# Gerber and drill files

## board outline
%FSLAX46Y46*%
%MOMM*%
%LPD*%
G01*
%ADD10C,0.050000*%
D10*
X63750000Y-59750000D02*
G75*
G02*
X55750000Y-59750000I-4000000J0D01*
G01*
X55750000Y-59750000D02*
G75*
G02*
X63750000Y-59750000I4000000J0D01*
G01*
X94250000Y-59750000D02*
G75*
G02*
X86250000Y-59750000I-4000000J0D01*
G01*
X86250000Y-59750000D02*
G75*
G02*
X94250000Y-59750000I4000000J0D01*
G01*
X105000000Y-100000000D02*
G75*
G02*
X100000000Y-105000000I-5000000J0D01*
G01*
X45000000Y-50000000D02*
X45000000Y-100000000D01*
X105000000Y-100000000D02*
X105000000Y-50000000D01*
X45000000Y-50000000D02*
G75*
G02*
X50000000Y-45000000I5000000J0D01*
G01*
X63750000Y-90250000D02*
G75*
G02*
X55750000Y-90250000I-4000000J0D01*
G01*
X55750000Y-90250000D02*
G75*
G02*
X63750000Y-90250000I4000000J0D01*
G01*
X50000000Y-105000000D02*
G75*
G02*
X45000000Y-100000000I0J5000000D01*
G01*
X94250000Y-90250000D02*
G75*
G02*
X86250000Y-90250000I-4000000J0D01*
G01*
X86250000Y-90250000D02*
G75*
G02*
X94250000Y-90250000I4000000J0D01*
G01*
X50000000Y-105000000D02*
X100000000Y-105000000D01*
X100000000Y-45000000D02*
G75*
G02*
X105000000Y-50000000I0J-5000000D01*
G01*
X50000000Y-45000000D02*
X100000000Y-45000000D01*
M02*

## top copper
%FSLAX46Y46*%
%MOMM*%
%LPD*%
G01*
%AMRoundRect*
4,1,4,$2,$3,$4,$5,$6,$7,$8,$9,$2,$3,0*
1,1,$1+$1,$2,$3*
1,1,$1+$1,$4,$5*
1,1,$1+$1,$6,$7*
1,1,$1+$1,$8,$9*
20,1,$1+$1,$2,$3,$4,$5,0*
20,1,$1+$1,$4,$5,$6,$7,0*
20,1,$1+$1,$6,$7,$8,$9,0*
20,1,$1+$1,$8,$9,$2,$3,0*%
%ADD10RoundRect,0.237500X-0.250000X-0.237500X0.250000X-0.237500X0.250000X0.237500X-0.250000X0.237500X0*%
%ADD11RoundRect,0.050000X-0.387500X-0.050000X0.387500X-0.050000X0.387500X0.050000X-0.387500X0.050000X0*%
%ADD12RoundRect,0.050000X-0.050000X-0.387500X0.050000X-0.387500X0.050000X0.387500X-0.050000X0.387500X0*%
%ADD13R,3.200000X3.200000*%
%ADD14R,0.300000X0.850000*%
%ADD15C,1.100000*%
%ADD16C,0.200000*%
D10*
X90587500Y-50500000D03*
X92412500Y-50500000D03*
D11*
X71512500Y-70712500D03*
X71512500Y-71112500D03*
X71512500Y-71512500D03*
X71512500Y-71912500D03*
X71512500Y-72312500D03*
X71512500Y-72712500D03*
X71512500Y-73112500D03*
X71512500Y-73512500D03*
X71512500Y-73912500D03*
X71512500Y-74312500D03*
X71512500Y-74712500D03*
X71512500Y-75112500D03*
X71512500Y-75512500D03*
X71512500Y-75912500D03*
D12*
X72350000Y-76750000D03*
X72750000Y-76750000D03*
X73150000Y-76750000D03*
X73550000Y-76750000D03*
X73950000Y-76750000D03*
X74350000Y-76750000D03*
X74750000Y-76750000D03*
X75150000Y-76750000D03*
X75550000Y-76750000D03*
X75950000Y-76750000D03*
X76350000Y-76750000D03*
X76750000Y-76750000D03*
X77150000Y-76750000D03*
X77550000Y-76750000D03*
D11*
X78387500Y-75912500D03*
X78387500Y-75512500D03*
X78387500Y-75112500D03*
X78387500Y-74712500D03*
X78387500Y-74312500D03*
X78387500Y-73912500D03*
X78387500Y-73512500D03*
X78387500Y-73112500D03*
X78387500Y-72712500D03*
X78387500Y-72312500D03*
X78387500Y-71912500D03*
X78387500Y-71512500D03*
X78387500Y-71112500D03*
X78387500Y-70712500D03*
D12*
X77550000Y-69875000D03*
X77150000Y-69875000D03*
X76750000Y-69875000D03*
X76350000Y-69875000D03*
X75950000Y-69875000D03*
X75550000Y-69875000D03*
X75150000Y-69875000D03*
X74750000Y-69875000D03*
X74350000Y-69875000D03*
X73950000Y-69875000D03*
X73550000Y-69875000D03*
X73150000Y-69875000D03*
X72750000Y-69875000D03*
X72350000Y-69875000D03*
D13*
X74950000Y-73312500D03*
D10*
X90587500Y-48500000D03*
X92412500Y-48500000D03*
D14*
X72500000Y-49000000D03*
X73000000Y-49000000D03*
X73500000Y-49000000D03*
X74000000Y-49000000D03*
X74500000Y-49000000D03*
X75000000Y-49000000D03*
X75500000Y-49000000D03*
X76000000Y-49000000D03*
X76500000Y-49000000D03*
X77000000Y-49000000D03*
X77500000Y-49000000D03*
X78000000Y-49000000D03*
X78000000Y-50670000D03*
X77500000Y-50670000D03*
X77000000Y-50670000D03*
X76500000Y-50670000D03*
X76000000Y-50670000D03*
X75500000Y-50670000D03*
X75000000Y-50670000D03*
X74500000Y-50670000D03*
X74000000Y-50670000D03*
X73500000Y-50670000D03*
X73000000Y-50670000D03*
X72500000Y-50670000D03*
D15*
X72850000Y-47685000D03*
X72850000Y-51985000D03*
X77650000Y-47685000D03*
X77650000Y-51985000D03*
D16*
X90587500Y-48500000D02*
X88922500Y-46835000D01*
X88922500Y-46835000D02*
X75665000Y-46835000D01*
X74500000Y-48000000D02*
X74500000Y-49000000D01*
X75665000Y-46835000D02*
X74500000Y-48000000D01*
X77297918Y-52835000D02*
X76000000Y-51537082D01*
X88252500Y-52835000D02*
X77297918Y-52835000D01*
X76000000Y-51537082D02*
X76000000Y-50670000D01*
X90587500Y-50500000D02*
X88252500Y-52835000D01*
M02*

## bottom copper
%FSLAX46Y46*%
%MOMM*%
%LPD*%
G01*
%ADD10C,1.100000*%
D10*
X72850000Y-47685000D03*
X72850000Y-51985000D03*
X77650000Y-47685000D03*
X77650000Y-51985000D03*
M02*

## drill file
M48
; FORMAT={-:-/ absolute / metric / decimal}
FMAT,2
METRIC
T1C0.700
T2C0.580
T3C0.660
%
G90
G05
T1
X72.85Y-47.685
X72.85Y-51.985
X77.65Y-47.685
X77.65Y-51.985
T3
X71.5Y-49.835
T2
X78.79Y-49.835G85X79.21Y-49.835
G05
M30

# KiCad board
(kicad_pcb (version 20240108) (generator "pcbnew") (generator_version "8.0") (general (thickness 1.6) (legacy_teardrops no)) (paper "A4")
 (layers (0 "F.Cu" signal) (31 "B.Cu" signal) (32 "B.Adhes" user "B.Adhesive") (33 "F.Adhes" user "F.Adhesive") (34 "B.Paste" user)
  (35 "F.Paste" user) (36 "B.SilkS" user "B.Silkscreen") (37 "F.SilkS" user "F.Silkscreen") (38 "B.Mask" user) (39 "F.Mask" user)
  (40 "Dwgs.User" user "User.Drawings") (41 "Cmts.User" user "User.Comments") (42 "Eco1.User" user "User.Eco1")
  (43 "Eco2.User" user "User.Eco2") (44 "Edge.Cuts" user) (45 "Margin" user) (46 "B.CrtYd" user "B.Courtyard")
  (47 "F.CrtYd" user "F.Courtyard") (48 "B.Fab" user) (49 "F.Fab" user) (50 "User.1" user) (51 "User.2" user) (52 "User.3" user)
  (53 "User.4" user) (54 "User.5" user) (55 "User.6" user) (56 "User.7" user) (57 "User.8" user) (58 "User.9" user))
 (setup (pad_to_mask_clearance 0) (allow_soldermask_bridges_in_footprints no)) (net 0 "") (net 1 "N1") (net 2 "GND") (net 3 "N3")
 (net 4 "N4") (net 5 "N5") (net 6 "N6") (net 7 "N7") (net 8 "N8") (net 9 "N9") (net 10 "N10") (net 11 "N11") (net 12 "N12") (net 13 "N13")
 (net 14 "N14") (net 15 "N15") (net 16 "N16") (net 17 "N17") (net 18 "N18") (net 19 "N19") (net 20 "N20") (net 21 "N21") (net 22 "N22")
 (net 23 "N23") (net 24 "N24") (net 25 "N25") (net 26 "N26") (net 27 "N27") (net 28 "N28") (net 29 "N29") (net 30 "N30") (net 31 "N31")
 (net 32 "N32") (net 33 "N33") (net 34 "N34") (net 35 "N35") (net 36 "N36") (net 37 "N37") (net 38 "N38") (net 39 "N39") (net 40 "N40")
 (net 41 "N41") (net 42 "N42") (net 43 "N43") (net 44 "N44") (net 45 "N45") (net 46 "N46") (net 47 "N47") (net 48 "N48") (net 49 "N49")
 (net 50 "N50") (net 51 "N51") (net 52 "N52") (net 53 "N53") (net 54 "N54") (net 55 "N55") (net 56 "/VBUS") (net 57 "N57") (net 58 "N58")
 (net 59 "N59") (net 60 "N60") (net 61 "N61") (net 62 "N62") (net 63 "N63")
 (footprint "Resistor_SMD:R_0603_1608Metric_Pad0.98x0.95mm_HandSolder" (layer "F.Cu") (at 91.5 50.5)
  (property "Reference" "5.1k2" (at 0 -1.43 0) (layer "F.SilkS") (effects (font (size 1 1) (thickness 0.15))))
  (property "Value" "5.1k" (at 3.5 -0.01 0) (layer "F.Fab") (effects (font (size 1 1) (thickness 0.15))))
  (pad "1" smd roundrect (at -0.9125 0) (size 0.975 0.95) (layers "F.Cu" "F.Paste" "F.Mask") (roundrect_rratio 0.25) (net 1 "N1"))
  (pad "2" smd roundrect (at 0.9125 0) (size 0.975 0.95) (layers "F.Cu" "F.Paste" "F.Mask") (roundrect_rratio 0.25) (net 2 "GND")))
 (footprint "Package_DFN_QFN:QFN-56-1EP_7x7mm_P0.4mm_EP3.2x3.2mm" (layer "F.Cu") (at 74.95 73.3125)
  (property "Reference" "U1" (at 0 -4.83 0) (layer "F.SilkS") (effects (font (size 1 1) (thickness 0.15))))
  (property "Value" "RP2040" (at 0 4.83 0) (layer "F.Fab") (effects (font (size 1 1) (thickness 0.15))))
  (pad "" smd roundrect (at -0.8 -0.8) (size 1.29 1.29) (layers "F.Paste") (roundrect_rratio 0.193798))
  (pad "" smd roundrect (at -0.8 0.8) (size 1.29 1.29) (layers "F.Paste") (roundrect_rratio 0.193798))
  (pad "" smd roundrect (at 0.8 -0.8) (size 1.29 1.29) (layers "F.Paste") (roundrect_rratio 0.193798))
  (pad "" smd roundrect (at 0.8 0.8) (size 1.29 1.29) (layers "F.Paste") (roundrect_rratio 0.193798))
  (pad "1" smd roundrect (at -3.4375 -2.6) (size 0.875 0.2) (layers "F.Cu" "F.Paste" "F.Mask") (roundrect_rratio 0.25) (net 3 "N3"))
  (pad "2" smd roundrect (at -3.4375 -2.2) (size 0.875 0.2) (layers "F.Cu" "F.Paste" "F.Mask") (roundrect_rratio 0.25) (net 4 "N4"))
  (pad "3" smd roundrect (at -3.4375 -1.8) (size 0.875 0.2) (layers "F.Cu" "F.Paste" "F.Mask") (roundrect_rratio 0.25) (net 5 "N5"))
  (pad "4" smd roundrect (at -3.4375 -1.4) (size 0.875 0.2) (layers "F.Cu" "F.Paste" "F.Mask") (roundrect_rratio 0.25) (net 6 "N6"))
  (pad "5" smd roundrect (at -3.4375 -1) (size 0.875 0.2) (layers "F.Cu" "F.Paste" "F.Mask") (roundrect_rratio 0.25) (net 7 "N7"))
  (pad "6" smd roundrect (at -3.4375 -0.6) (size 0.875 0.2) (layers "F.Cu" "F.Paste" "F.Mask") (roundrect_rratio 0.25) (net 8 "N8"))
  (pad "7" smd roundrect (at -3.4375 -0.2) (size 0.875 0.2) (layers "F.Cu" "F.Paste" "F.Mask") (roundrect_rratio 0.25) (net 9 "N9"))
  (pad "8" smd roundrect (at -3.4375 0.2) (size 0.875 0.2) (layers "F.Cu" "F.Paste" "F.Mask") (roundrect_rratio 0.25) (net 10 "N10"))
  (pad "9" smd roundrect (at -3.4375 0.6) (size 0.875 0.2) (layers "F.Cu" "F.Paste" "F.Mask") (roundrect_rratio 0.25) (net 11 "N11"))
  (pad "10" smd roundrect (at -3.4375 1) (size 0.875 0.2) (layers "F.Cu" "F.Paste" "F.Mask") (roundrect_rratio 0.25) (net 3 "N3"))
  (pad "11" smd roundrect (at -3.4375 1.4) (size 0.875 0.2) (layers "F.Cu" "F.Paste" "F.Mask") (roundrect_rratio 0.25) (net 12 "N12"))
  (pad "12" smd roundrect (at -3.4375 1.8) (size 0.875 0.2) (layers "F.Cu" "F.Paste" "F.Mask") (roundrect_rratio 0.25) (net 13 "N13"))
  (pad "13" smd roundrect (at -3.4375 2.2) (size 0.875 0.2) (layers "F.Cu" "F.Paste" "F.Mask") (roundrect_rratio 0.25) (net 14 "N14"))
  (pad "14" smd roundrect (at -3.4375 2.6) (size 0.875 0.2) (layers "F.Cu" "F.Paste" "F.Mask") (roundrect_rratio 0.25) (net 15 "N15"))
  (pad "15" smd roundrect (at -2.6 3.4375) (size 0.2 0.875) (layers "F.Cu" "F.Paste" "F.Mask") (roundrect_rratio 0.25) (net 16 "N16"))
  (pad "16" smd roundrect (at -2.2 3.4375) (size 0.2 0.875) (layers "F.Cu" "F.Paste" "F.Mask") (roundrect_rratio 0.25) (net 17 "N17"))
  (pad "17" smd roundrect (at -1.8 3.4375) (size 0.2 0.875) (layers "F.Cu" "F.Paste" "F.Mask") (roundrect_rratio 0.25) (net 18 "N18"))
  (pad "18" smd roundrect (at -1.4 3.4375) (size 0.2 0.875) (layers "F.Cu" "F.Paste" "F.Mask") (roundrect_rratio 0.25) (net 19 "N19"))
  (pad "19" smd roundrect (at -1 3.4375) (size 0.2 0.875) (layers "F.Cu" "F.Paste" "F.Mask") (roundrect_rratio 0.25) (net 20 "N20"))
  (pad "20" smd roundrect (at -0.6 3.4375) (size 0.2 0.875) (layers "F.Cu" "F.Paste" "F.Mask") (roundrect_rratio 0.25) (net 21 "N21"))
  (pad "21" smd roundrect (at -0.2 3.4375) (size 0.2 0.875) (layers "F.Cu" "F.Paste" "F.Mask") (roundrect_rratio 0.25) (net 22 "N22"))
  (pad "22" smd roundrect (at 0.2 3.4375) (size 0.2 0.875) (layers "F.Cu" "F.Paste" "F.Mask") (roundrect_rratio 0.25) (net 3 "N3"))
  (pad "23" smd roundrect (at 0.6 3.4375) (size 0.2 0.875) (layers "F.Cu" "F.Paste" "F.Mask") (roundrect_rratio 0.25) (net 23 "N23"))
  (pad "24" smd roundrect (at 1 3.4375) (size 0.2 0.875) (layers "F.Cu" "F.Paste" "F.Mask") (roundrect_rratio 0.25) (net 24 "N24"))
  (pad "25" smd roundrect (at 1.4 3.4375) (size 0.2 0.875) (layers "F.Cu" "F.Paste" "F.Mask") (roundrect_rratio 0.25) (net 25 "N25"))
  (pad "26" smd roundrect (at 1.8 3.4375) (size 0.2 0.875) (layers "F.Cu" "F.Paste" "F.Mask") (roundrect_rratio 0.25) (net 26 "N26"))
  (pad "27" smd roundrect (at 2.2 3.4375) (size 0.2 0.875) (layers "F.Cu" "F.Paste" "F.Mask") (roundrect_rratio 0.25) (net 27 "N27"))
  (pad "28" smd roundrect (at 2.6 3.4375) (size 0.2 0.875) (layers "F.Cu" "F.Paste" "F.Mask") (roundrect_rratio 0.25) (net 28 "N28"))
  (pad "29" smd roundrect (at 3.4375 2.6) (size 0.875 0.2) (layers "F.Cu" "F.Paste" "F.Mask") (roundrect_rratio 0.25) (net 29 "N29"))
  (pad "30" smd roundrect (at 3.4375 2.2) (size 0.875 0.2) (layers "F.Cu" "F.Paste" "F.Mask") (roundrect_rratio 0.25) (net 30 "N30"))
  (pad "31" smd roundrect (at 3.4375 1.8) (size 0.875 0.2) (layers "F.Cu" "F.Paste" "F.Mask") (roundrect_rratio 0.25) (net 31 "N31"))
  (pad "32" smd roundrect (at 3.4375 1.4) (size 0.875 0.2) (layers "F.Cu" "F.Paste" "F.Mask") (roundrect_rratio 0.25) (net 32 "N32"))
  (pad "33" smd roundrect (at 3.4375 1) (size 0.875 0.2) (layers "F.Cu" "F.Paste" "F.Mask") (roundrect_rratio 0.25) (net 3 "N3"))
  (pad "34" smd roundrect (at 3.4375 0.6) (size 0.875 0.2) (layers "F.Cu" "F.Paste" "F.Mask") (roundrect_rratio 0.25) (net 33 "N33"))
  (pad "35" smd roundrect (at 3.4375 0.2) (size 0.875 0.2) (layers "F.Cu" "F.Paste" "F.Mask") (roundrect_rratio 0.25) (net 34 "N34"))
  (pad "36" smd roundrect (at 3.4375 -0.2) (size 0.875 0.2) (layers "F.Cu" "F.Paste" "F.Mask") (roundrect_rratio 0.25) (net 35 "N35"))
  (pad "37" smd roundrect (at 3.4375 -0.6) (size 0.875 0.2) (layers "F.Cu" "F.Paste" "F.Mask") (roundrect_rratio 0.25) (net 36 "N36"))
  (pad "38" smd roundrect (at 3.4375 -1) (size 0.875 0.2) (layers "F.Cu" "F.Paste" "F.Mask") (roundrect_rratio 0.25) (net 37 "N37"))
  (pad "39" smd roundrect (at 3.4375 -1.4) (size 0.875 0.2) (layers "F.Cu" "F.Paste" "F.Mask") (roundrect_rratio 0.25) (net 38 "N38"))
  (pad "40" smd roundrect (at 3.4375 -1.8) (size 0.875 0.2) (layers "F.Cu" "F.Paste" "F.Mask") (roundrect_rratio 0.25) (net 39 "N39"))
  (pad "41" smd roundrect (at 3.4375 -2.2) (size 0.875 0.2) (layers "F.Cu" "F.Paste" "F.Mask") (roundrect_rratio 0.25) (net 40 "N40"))
  (pad "42" smd roundrect (at 3.4375 -2.6) (size 0.875 0.2) (layers "F.Cu" "F.Paste" "F.Mask") (roundrect_rratio 0.25) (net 3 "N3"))
  (pad "43" smd roundrect (at 2.6 -3.4375) (size 0.2 0.875) (layers "F.Cu" "F.Paste" "F.Mask") (roundrect_rratio 0.25) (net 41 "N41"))
  (pad "44" smd roundrect (at 2.2 -3.4375) (size 0.2 0.875) (layers "F.Cu" "F.Paste" "F.Mask") (roundrect_rratio 0.25) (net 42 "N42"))
  (pad "45" smd roundrect (at 1.8 -3.4375) (size 0.2 0.875) (layers "F.Cu" "F.Paste" "F.Mask") (roundrect_rratio 0.25) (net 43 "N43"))
  (pad "46" smd roundrect (at 1.4 -3.4375) (size 0.2 0.875) (layers "F.Cu" "F.Paste" "F.Mask") (roundrect_rratio 0.25) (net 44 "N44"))
  (pad "47" smd roundrect (at 1 -3.4375) (size 0.2 0.875) (layers "F.Cu" "F.Paste" "F.Mask") (roundrect_rratio 0.25) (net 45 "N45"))
  (pad "48" smd roundrect (at 0.6 -3.4375) (size 0.2 0.875) (layers "F.Cu" "F.Paste" "F.Mask") (roundrect_rratio 0.25) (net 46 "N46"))
  (pad "49" smd roundrect (at 0.2 -3.4375) (size 0.2 0.875) (layers "F.Cu" "F.Paste" "F.Mask") (roundrect_rratio 0.25) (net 3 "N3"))
  (pad "50" smd roundrect (at -0.2 -3.4375) (size 0.2 0.875) (layers "F.Cu" "F.Paste" "F.Mask") (roundrect_rratio 0.25) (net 23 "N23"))
  (pad "51" smd roundrect (at -0.6 -3.4375) (size 0.2 0.875) (layers "F.Cu" "F.Paste" "F.Mask") (roundrect_rratio 0.25) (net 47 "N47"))
  (pad "52" smd roundrect (at -1 -3.4375) (size 0.2 0.875) (layers "F.Cu" "F.Paste" "F.Mask") (roundrect_rratio 0.25) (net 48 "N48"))
  (pad "53" smd roundrect (at -1.4 -3.4375) (size 0.2 0.875) (layers "F.Cu" "F.Paste" "F.Mask") (roundrect_rratio 0.25) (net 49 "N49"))
  (pad "54" smd roundrect (at -1.8 -3.4375) (size 0.2 0.875) (layers "F.Cu" "F.Paste" "F.Mask") (roundrect_rratio 0.25) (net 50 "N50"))
  (pad "55" smd roundrect (at -2.2 -3.4375) (size 0.2 0.875) (layers "F.Cu" "F.Paste" "F.Mask") (roundrect_rratio 0.25) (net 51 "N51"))
  (pad "56" smd roundrect (at -2.6 -3.4375) (size 0.2 0.875) (layers "F.Cu" "F.Paste" "F.Mask") (roundrect_rratio 0.25) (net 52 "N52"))
  (pad "57" smd rect (at 0 0) (size 3.2 3.2) (layers "F.Cu" "F.Mask") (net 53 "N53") (zone_connect 2)))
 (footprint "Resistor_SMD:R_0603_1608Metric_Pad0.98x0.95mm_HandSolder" (layer "F.Cu") (at 91.5 48.5)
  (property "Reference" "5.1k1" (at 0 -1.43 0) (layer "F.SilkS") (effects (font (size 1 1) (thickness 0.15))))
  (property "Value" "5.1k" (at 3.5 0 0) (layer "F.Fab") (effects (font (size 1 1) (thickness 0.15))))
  (pad "1" smd roundrect (at -0.9125 0) (size 0.975 0.95) (layers "F.Cu" "F.Paste" "F.Mask") (roundrect_rratio 0.25) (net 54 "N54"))
  (pad "2" smd roundrect (at 0.9125 0) (size 0.975 0.95) (layers "F.Cu" "F.Paste" "F.Mask") (roundrect_rratio 0.25) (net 2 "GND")))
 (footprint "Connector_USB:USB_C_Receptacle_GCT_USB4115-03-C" (layer "F.Cu") (at 75.25 49.835)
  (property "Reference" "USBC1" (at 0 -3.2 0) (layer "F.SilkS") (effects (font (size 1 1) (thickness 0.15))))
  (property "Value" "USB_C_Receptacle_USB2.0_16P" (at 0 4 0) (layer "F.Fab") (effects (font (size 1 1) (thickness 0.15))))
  (pad "" np_thru_hole circle (at -3.75 0) (size 0.66 0.66) (drill 0.66) (layers "F&B.Cu" "*.Mask"))
  (pad "" np_thru_hole oval (at 3.75 0) (size 1 0.58) (drill oval 1 0.58) (layers "F&B.Cu" "*.Mask"))
  (pad "A1" smd rect (at -2.75 -0.835) (size 0.3 0.85) (layers "F.Cu" "F.Paste" "F.Mask") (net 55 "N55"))
  (pad "A2" smd rect (at -2.25 -0.835) (size 0.3 0.85) (layers "F.Cu" "F.Paste" "F.Mask"))
  (pad "A3" smd rect (at -1.75 -0.835) (size 0.3 0.85) (layers "F.Cu" "F.Paste" "F.Mask"))
  (pad "A4" smd rect (at -1.25 -0.835) (size 0.3 0.85) (layers "F.Cu" "F.Paste" "F.Mask") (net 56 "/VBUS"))
  (pad "A5" smd rect (at -0.75 -0.835) (size 0.3 0.85) (layers "F.Cu" "F.Paste" "F.Mask") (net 54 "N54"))
  (pad "A6" smd rect (at -0.25 -0.835) (size 0.3 0.85) (layers "F.Cu" "F.Paste" "F.Mask") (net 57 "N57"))
  (pad "A7" smd rect (at 0.25 -0.835) (size 0.3 0.85) (layers "F.Cu" "F.Paste" "F.Mask") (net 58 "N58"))
  (pad "A8" smd rect (at 0.75 -0.835) (size 0.3 0.85) (layers "F.Cu" "F.Paste" "F.Mask") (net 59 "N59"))
  (pad "A9" smd rect (at 1.25 -0.835) (size 0.3 0.85) (layers "F.Cu" "F.Paste" "F.Mask") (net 56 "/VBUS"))
  (pad "A10" smd rect (at 1.75 -0.835) (size 0.3 0.85) (layers "F.Cu" "F.Paste" "F.Mask"))
  (pad "A11" smd rect (at 2.25 -0.835) (size 0.3 0.85) (layers "F.Cu" "F.Paste" "F.Mask"))
  (pad "A12" smd rect (at 2.75 -0.835) (size 0.3 0.85) (layers "F.Cu" "F.Paste" "F.Mask") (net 55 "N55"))
  (pad "B1" smd rect (at 2.75 0.835) (size 0.3 0.85) (layers "F.Cu" "F.Paste" "F.Mask") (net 55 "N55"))
  (pad "B2" smd rect (at 2.25 0.835) (size 0.3 0.85) (layers "F.Cu" "F.Paste" "F.Mask"))
  (pad "B3" smd rect (at 1.75 0.835) (size 0.3 0.85) (layers "F.Cu" "F.Paste" "F.Mask"))
  (pad "B4" smd rect (at 1.25 0.835) (size 0.3 0.85) (layers "F.Cu" "F.Paste" "F.Mask") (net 56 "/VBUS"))
  (pad "B5" smd rect (at 0.75 0.835) (size 0.3 0.85) (layers "F.Cu" "F.Paste" "F.Mask") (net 1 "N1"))
  (pad "B6" smd rect (at 0.25 0.835) (size 0.3 0.85) (layers "F.Cu" "F.Paste" "F.Mask") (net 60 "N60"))
  (pad "B7" smd rect (at -0.25 0.835) (size 0.3 0.85) (layers "F.Cu" "F.Paste" "F.Mask") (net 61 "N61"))
  (pad "B8" smd rect (at -0.75 0.835) (size 0.3 0.85) (layers "F.Cu" "F.Paste" "F.Mask") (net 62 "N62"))
  (pad "B9" smd rect (at -1.25 0.835) (size 0.3 0.85) (layers "F.Cu" "F.Paste" "F.Mask") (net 56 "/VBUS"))
  (pad "B10" smd rect (at -1.75 0.835) (size 0.3 0.85) (layers "F.Cu" "F.Paste" "F.Mask"))
  (pad "B11" smd rect (at -2.25 0.835) (size 0.3 0.85) (layers "F.Cu" "F.Paste" "F.Mask"))
  (pad "B12" smd rect (at -2.75 0.835) (size 0.3 0.85) (layers "F.Cu" "F.Paste" "F.Mask") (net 55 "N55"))
  (pad "S1" thru_hole circle (at -2.4 -2.15) (size 1.1 1.1) (drill 0.7) (layers "*.Cu" "*.Mask" "F.Paste") (remove_unused_layers no)
   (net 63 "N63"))
  (pad "S1" thru_hole circle (at -2.4 2.15) (size 1.1 1.1) (drill 0.7) (layers "*.Cu" "*.Mask" "F.Paste") (remove_unused_layers no)
   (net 63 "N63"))
  (pad "S1" thru_hole circle (at 2.4 -2.15) (size 1.1 1.1) (drill 0.7) (layers "*.Cu" "*.Mask" "F.Paste") (remove_unused_layers no)
   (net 63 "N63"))
  (pad "S1" thru_hole circle (at 2.4 2.15) (size 1.1 1.1) (drill 0.7) (layers "*.Cu" "*.Mask" "F.Paste") (remove_unused_layers no)
   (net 63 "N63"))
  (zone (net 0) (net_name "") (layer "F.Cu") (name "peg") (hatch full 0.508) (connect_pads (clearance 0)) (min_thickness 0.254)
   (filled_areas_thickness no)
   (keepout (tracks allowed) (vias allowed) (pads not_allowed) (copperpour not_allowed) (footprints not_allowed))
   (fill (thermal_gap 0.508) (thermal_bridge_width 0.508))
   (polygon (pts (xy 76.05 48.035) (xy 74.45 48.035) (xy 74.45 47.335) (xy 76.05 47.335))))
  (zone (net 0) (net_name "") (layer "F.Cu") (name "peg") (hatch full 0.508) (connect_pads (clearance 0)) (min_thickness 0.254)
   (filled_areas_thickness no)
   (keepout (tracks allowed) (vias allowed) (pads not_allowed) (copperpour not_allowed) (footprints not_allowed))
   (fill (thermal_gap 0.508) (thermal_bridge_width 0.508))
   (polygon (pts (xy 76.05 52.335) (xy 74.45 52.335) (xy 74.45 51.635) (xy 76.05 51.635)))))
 (gr_circle (center 59.75 59.75) (end 63.75 59.75) (stroke (width 0.05) (type default)) (fill none) (layer "Edge.Cuts"))
 (gr_circle (center 90.25 59.75) (end 94.25 59.75) (stroke (width 0.05) (type default)) (fill none) (layer "Edge.Cuts"))
 (gr_arc (start 105 100) (mid 103.535534 103.535534) (end 100 105) (stroke (width 0.05) (type default)) (layer "Edge.Cuts"))
 (gr_line (start 45 50) (end 45 100) (stroke (width 0.05) (type default)) (layer "Edge.Cuts"))
 (gr_line (start 105 100) (end 105 50) (stroke (width 0.05) (type default)) (layer "Edge.Cuts"))
 (gr_arc (start 45 50) (mid 46.464466 46.464466) (end 50 45) (stroke (width 0.05) (type default)) (layer "Edge.Cuts"))
 (gr_circle (center 59.75 90.25) (end 63.75 90.25) (stroke (width 0.05) (type default)) (fill none) (layer "Edge.Cuts"))
 (gr_arc (start 50 105) (mid 46.464466 103.535534) (end 45 100) (stroke (width 0.05) (type default)) (layer "Edge.Cuts"))
 (gr_circle (center 90.25 90.25) (end 94.25 90.25) (stroke (width 0.05) (type default)) (fill none) (layer "Edge.Cuts"))
 (gr_line (start 50 105) (end 100 105) (stroke (width 0.05) (type default)) (layer "Edge.Cuts"))
 (gr_arc (start 100 45) (mid 103.535534 46.464466) (end 105 50) (stroke (width 0.05) (type default)) (layer "Edge.Cuts"))
 (gr_line (start 50 45) (end 100 45) (stroke (width 0.05) (type default)) (layer "Edge.Cuts"))
 (segment (start 90.5875 48.5) (end 88.9225 46.835) (width 0.2) (layer "F.Cu") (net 54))
 (segment (start 88.9225 46.835) (end 75.665 46.835) (width 0.2) (layer "F.Cu") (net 54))
 (segment (start 74.5 48) (end 74.5 49) (width 0.2) (layer "F.Cu") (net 54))
 (segment (start 75.665 46.835) (end 74.5 48) (width 0.2) (layer "F.Cu") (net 54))
 (segment (start 77.297918 52.835) (end 76 51.537082) (width 0.2) (layer "F.Cu") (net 1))
 (segment (start 88.2525 52.835) (end 77.297918 52.835) (width 0.2) (layer "F.Cu") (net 1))
 (segment (start 76 51.537082) (end 76 50.67) (width 0.2) (layer "F.Cu") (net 1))
 (segment (start 90.5875 50.5) (end 88.2525 52.835) (width 0.2) (layer "F.Cu") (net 1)))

